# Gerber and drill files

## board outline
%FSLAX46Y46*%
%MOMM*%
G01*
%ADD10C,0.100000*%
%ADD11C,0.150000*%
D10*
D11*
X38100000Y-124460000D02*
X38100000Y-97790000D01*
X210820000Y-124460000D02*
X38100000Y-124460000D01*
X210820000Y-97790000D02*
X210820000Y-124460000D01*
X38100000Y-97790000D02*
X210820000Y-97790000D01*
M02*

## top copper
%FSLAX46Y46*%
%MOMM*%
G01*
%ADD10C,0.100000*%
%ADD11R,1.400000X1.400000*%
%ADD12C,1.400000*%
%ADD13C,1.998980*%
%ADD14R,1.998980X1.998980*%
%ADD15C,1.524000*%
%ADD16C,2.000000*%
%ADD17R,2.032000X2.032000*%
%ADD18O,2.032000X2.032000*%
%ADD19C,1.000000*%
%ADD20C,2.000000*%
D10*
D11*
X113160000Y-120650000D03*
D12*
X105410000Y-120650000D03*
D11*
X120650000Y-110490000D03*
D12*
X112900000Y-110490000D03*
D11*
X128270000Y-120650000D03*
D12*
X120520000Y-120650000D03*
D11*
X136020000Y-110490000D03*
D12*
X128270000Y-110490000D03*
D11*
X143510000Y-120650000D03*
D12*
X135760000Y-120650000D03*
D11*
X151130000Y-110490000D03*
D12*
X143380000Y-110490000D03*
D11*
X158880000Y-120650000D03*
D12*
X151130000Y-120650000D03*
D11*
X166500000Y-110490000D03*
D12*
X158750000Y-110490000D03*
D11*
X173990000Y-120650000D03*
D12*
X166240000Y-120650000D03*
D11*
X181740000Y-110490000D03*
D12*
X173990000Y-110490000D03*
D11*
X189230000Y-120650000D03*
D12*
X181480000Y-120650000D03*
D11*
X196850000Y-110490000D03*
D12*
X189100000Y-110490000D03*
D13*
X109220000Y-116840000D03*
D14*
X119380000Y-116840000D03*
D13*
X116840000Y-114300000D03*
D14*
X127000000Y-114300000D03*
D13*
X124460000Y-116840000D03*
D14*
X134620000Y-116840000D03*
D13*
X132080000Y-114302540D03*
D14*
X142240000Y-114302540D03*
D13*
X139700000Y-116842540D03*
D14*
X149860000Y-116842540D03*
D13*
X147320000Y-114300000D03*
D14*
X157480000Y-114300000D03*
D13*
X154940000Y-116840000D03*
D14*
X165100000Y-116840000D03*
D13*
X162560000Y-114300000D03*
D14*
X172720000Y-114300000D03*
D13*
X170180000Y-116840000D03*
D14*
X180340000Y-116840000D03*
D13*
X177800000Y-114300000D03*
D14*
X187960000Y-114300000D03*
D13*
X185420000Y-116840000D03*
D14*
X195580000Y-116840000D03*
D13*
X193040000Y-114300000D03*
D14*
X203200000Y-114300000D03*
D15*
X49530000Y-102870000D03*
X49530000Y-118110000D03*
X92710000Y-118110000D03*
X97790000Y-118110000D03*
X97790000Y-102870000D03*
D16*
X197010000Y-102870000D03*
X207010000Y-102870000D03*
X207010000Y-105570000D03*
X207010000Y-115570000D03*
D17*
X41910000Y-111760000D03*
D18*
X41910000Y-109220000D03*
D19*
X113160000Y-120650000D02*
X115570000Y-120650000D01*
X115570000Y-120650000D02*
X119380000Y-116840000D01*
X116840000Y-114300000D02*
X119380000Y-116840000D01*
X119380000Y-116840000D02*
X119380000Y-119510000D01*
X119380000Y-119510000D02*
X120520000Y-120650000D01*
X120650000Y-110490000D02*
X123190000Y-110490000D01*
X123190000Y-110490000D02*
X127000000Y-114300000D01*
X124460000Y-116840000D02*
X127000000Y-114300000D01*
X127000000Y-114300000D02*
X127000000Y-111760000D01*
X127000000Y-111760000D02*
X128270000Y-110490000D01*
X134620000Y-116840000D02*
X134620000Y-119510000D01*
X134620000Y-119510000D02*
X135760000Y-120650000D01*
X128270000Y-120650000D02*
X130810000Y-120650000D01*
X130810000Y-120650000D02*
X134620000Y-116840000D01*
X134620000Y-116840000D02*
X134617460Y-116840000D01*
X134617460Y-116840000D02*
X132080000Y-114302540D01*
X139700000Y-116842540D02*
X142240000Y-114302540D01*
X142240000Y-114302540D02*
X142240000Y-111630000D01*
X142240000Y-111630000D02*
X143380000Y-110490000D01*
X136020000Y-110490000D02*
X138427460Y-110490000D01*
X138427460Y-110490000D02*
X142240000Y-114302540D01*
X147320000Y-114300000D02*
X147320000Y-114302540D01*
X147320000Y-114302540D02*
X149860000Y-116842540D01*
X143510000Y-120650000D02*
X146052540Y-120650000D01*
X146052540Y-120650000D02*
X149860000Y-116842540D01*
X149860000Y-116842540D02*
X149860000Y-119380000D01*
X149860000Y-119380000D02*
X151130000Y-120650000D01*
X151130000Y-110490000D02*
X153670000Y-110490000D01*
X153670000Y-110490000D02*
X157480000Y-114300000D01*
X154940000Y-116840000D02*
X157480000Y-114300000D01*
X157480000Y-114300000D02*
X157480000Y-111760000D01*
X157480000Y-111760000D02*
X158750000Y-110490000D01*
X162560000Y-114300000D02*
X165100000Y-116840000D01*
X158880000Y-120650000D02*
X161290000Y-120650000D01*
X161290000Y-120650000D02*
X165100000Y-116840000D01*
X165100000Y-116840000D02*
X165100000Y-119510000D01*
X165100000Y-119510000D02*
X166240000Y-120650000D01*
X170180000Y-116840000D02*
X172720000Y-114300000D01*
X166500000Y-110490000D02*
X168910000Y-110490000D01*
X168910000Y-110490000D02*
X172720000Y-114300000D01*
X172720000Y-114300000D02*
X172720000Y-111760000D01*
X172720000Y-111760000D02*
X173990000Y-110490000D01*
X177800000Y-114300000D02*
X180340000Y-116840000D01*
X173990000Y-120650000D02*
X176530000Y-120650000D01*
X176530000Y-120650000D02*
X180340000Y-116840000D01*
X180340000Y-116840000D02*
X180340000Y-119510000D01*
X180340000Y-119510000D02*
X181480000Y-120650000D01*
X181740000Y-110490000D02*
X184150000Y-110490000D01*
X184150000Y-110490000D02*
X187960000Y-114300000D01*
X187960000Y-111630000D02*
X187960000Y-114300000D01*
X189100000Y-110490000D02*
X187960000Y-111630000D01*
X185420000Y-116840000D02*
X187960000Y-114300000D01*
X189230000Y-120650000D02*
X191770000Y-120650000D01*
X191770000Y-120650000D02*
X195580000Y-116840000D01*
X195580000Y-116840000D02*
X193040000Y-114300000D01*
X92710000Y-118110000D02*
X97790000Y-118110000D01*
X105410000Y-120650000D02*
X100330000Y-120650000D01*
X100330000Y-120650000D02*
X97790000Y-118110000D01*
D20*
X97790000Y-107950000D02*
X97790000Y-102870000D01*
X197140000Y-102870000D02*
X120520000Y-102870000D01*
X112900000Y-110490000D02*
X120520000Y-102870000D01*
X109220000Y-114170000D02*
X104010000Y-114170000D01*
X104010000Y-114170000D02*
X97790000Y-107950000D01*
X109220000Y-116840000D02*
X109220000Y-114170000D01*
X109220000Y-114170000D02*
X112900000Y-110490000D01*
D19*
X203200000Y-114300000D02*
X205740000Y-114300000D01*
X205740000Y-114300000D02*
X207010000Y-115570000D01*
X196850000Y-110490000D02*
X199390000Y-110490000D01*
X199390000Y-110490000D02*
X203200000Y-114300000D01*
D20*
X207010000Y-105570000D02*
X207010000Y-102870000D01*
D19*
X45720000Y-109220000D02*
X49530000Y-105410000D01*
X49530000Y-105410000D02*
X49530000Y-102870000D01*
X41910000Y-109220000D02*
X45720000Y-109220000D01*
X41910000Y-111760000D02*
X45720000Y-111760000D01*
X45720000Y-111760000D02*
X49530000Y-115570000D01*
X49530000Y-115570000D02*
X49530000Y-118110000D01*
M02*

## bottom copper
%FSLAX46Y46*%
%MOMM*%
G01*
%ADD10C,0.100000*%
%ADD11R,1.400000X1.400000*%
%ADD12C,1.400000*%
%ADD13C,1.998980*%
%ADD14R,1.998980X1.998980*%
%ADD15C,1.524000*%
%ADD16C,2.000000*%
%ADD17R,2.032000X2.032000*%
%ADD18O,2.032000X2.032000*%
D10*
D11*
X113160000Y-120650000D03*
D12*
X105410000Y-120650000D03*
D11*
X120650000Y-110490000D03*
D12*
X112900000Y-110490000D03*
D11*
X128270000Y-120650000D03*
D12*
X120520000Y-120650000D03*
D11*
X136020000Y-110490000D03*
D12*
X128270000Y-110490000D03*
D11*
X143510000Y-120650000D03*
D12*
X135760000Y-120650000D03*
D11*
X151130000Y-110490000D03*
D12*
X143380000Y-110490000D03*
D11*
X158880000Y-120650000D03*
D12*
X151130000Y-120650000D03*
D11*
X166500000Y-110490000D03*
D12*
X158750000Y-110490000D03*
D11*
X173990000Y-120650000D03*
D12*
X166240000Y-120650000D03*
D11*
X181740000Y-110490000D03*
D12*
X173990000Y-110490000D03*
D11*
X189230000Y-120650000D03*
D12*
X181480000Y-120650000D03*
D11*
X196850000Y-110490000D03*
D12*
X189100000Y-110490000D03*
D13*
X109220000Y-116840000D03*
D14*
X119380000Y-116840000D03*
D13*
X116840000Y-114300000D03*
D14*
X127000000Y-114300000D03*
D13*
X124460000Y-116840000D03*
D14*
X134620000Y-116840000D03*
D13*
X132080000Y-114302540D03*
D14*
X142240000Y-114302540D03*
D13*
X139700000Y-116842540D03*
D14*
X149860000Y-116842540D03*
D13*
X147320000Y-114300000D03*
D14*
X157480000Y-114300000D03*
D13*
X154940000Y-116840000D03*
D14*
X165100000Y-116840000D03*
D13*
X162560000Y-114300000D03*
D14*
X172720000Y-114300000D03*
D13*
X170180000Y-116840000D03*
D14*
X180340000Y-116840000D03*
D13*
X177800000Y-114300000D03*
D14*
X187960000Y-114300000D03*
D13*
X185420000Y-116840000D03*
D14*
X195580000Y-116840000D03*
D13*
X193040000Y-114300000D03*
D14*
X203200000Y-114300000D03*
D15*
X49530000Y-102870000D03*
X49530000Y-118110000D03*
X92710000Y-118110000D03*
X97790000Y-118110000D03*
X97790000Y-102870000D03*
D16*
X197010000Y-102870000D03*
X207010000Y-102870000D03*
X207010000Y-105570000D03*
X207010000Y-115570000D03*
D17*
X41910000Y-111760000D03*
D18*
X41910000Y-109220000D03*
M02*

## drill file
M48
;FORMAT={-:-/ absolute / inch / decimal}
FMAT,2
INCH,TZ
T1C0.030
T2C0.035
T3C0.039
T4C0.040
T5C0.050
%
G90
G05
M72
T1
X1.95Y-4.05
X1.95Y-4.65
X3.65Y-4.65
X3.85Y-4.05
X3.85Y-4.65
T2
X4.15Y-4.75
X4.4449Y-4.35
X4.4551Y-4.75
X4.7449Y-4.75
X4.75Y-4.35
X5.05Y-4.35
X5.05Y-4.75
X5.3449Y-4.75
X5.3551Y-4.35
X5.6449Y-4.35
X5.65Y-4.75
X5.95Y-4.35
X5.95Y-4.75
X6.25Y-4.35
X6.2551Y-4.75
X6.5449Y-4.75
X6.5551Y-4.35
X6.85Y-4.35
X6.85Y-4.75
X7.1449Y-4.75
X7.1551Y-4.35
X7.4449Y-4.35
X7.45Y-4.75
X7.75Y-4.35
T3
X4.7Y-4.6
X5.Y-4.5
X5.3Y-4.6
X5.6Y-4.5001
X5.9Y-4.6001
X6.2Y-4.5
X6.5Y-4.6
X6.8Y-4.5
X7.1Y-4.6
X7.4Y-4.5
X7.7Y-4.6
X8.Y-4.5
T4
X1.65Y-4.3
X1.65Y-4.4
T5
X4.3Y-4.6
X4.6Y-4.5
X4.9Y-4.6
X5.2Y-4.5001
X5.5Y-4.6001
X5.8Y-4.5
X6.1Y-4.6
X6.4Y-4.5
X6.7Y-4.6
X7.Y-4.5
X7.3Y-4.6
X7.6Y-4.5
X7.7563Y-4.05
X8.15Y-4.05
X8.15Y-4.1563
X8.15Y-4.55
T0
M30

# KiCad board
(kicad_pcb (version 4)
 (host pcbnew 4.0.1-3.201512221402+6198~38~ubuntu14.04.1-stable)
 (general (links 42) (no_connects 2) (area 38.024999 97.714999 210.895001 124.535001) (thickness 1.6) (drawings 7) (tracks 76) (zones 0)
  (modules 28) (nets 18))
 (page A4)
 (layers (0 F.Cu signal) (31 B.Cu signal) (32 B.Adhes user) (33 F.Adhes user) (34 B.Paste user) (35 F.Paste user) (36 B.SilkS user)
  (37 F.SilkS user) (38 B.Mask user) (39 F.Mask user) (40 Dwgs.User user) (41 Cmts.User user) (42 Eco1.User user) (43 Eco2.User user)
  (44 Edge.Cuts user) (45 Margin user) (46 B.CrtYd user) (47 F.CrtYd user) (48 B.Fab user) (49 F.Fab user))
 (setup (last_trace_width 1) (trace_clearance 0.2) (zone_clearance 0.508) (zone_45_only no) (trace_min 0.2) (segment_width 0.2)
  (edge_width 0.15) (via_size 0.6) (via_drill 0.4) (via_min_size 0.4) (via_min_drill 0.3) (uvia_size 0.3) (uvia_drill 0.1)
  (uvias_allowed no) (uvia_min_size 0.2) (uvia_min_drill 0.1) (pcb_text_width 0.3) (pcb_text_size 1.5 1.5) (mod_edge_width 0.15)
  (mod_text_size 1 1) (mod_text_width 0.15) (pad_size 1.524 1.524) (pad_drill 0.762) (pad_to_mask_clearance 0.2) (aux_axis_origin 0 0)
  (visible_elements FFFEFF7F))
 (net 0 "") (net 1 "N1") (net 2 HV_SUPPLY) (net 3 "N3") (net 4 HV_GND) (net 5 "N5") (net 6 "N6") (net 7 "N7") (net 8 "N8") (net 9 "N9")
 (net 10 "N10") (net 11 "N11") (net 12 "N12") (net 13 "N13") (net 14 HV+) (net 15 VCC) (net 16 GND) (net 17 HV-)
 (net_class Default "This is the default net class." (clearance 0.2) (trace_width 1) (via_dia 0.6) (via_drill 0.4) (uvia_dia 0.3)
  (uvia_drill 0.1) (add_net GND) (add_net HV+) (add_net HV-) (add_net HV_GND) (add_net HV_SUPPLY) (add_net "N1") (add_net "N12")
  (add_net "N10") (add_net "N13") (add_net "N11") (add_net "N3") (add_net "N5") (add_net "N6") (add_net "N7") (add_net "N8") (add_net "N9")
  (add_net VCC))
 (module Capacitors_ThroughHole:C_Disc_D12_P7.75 (layer F.Cu) (at 113.16 120.65 180)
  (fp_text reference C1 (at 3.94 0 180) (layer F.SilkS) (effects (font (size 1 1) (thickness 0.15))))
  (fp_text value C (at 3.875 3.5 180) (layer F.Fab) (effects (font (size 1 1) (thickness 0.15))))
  (pad 1 thru_hole rect (at 0 0 180) (size 1.4 1.4) (drill 0.9) (layers *.Cu *.Mask F.SilkS) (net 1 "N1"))
  (pad 2 thru_hole circle (at 7.75 0 180) (size 1.4 1.4) (drill 0.9) (layers *.Cu *.Mask F.SilkS) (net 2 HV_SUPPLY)))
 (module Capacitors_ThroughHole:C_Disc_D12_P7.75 (layer F.Cu) (at 120.65 110.49 180)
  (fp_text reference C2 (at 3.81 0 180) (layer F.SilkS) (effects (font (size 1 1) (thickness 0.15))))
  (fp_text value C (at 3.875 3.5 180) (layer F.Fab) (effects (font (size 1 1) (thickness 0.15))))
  (pad 1 thru_hole rect (at 0 0 180) (size 1.4 1.4) (drill 0.9) (layers *.Cu *.Mask F.SilkS) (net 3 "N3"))
  (pad 2 thru_hole circle (at 7.75 0 180) (size 1.4 1.4) (drill 0.9) (layers *.Cu *.Mask F.SilkS) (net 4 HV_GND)))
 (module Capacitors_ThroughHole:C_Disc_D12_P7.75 (layer F.Cu) (at 128.27 120.65 180)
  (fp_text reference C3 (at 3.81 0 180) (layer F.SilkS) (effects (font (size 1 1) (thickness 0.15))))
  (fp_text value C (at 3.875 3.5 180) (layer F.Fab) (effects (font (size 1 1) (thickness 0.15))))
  (pad 1 thru_hole rect (at 0 0 180) (size 1.4 1.4) (drill 0.9) (layers *.Cu *.Mask F.SilkS) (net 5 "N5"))
  (pad 2 thru_hole circle (at 7.75 0 180) (size 1.4 1.4) (drill 0.9) (layers *.Cu *.Mask F.SilkS) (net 1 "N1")))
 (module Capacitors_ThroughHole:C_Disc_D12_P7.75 (layer F.Cu) (at 136.02 110.49 180)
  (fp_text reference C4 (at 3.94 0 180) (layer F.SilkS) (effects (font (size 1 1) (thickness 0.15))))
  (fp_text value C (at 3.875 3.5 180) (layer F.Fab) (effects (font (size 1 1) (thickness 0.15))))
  (pad 1 thru_hole rect (at 0 0 180) (size 1.4 1.4) (drill 0.9) (layers *.Cu *.Mask F.SilkS) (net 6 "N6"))
  (pad 2 thru_hole circle (at 7.75 0 180) (size 1.4 1.4) (drill 0.9) (layers *.Cu *.Mask F.SilkS) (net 3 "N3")))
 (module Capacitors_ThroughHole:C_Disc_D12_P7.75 (layer F.Cu) (at 143.51 120.65 180)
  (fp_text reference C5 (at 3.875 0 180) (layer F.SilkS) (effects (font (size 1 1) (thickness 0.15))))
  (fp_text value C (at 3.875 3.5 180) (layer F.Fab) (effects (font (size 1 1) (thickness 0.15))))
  (pad 1 thru_hole rect (at 0 0 180) (size 1.4 1.4) (drill 0.9) (layers *.Cu *.Mask F.SilkS) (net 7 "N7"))
  (pad 2 thru_hole circle (at 7.75 0 180) (size 1.4 1.4) (drill 0.9) (layers *.Cu *.Mask F.SilkS) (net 5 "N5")))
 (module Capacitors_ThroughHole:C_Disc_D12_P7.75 (layer F.Cu) (at 151.13 110.49 180)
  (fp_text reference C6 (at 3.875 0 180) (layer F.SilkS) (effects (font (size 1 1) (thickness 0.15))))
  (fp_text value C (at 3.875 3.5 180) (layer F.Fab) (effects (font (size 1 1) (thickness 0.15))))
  (pad 1 thru_hole rect (at 0 0 180) (size 1.4 1.4) (drill 0.9) (layers *.Cu *.Mask F.SilkS) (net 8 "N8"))
  (pad 2 thru_hole circle (at 7.75 0 180) (size 1.4 1.4) (drill 0.9) (layers *.Cu *.Mask F.SilkS) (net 6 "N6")))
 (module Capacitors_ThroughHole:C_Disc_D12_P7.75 (layer F.Cu) (at 158.88 120.65 180)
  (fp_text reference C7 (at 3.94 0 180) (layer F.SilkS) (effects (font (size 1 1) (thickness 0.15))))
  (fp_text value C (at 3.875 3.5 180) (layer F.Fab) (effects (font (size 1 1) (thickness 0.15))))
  (pad 1 thru_hole rect (at 0 0 180) (size 1.4 1.4) (drill 0.9) (layers *.Cu *.Mask F.SilkS) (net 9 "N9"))
  (pad 2 thru_hole circle (at 7.75 0 180) (size 1.4 1.4) (drill 0.9) (layers *.Cu *.Mask F.SilkS) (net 7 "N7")))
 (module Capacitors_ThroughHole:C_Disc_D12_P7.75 (layer F.Cu) (at 166.5 110.49 180)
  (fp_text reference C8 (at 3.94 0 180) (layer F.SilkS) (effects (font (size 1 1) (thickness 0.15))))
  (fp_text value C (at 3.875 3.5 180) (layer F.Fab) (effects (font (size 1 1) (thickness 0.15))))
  (pad 1 thru_hole rect (at 0 0 180) (size 1.4 1.4) (drill 0.9) (layers *.Cu *.Mask F.SilkS) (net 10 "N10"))
  (pad 2 thru_hole circle (at 7.75 0 180) (size 1.4 1.4) (drill 0.9) (layers *.Cu *.Mask F.SilkS) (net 8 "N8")))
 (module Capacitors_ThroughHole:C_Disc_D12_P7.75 (layer F.Cu) (at 173.99 120.65 180)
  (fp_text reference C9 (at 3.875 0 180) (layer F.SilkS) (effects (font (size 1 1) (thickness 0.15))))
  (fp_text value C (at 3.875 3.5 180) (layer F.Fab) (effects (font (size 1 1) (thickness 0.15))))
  (pad 1 thru_hole rect (at 0 0 180) (size 1.4 1.4) (drill 0.9) (layers *.Cu *.Mask F.SilkS) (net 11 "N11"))
  (pad 2 thru_hole circle (at 7.75 0 180) (size 1.4 1.4) (drill 0.9) (layers *.Cu *.Mask F.SilkS) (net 9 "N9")))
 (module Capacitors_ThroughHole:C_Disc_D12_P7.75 (layer F.Cu) (at 181.74 110.49 180)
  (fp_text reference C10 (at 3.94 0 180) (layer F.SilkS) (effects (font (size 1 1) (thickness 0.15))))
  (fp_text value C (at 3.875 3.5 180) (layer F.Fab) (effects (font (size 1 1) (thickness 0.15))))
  (pad 1 thru_hole rect (at 0 0 180) (size 1.4 1.4) (drill 0.9) (layers *.Cu *.Mask F.SilkS) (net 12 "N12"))
  (pad 2 thru_hole circle (at 7.75 0 180) (size 1.4 1.4) (drill 0.9) (layers *.Cu *.Mask F.SilkS) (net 10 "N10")))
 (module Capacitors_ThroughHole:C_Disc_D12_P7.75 (layer F.Cu) (at 189.23 120.65 180)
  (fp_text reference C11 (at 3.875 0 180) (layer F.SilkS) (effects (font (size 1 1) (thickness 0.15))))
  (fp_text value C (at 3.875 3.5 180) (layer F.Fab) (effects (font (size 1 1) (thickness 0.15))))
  (pad 1 thru_hole rect (at 0 0 180) (size 1.4 1.4) (drill 0.9) (layers *.Cu *.Mask F.SilkS) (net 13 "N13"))
  (pad 2 thru_hole circle (at 7.75 0 180) (size 1.4 1.4) (drill 0.9) (layers *.Cu *.Mask F.SilkS) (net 11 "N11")))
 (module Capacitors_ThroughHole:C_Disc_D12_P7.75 (layer F.Cu) (at 196.85 110.49 180)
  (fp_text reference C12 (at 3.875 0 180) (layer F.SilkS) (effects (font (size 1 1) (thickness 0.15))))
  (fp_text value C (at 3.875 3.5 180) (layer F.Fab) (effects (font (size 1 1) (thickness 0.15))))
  (pad 1 thru_hole rect (at 0 0 180) (size 1.4 1.4) (drill 0.9) (layers *.Cu *.Mask F.SilkS) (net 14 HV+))
  (pad 2 thru_hole circle (at 7.75 0 180) (size 1.4 1.4) (drill 0.9) (layers *.Cu *.Mask F.SilkS) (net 12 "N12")))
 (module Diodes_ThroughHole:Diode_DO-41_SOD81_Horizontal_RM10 (layer F.Cu) (at 119.38 116.83746 180)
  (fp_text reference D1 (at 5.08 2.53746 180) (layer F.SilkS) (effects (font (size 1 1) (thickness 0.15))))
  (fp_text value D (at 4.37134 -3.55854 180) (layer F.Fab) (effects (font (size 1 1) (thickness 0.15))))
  (pad 2 thru_hole circle (at 10.16 -0.00254) (size 1.99898 1.99898) (drill 1.27) (layers *.Cu *.Mask F.SilkS) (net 4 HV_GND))
  (pad 1 thru_hole rect (at 0 -0.00254) (size 1.99898 1.99898) (drill 1.00076) (layers *.Cu *.Mask F.SilkS) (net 1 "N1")))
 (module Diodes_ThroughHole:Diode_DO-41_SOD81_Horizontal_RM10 (layer F.Cu) (at 127 114.29746 180)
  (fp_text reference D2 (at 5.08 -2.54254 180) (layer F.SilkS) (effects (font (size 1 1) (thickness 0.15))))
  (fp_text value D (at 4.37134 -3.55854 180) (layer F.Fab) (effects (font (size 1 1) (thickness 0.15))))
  (pad 2 thru_hole circle (at 10.16 -0.00254) (size 1.99898 1.99898) (drill 1.27) (layers *.Cu *.Mask F.SilkS) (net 1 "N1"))
  (pad 1 thru_hole rect (at 0 -0.00254) (size 1.99898 1.99898) (drill 1.00076) (layers *.Cu *.Mask F.SilkS) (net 3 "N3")))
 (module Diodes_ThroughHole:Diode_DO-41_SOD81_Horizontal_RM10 (layer F.Cu) (at 134.62 116.83746 180)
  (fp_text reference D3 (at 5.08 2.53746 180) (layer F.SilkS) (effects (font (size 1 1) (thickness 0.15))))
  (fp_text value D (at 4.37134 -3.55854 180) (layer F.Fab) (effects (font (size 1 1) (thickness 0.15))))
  (pad 2 thru_hole circle (at 10.16 -0.00254) (size 1.99898 1.99898) (drill 1.27) (layers *.Cu *.Mask F.SilkS) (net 3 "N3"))
  (pad 1 thru_hole rect (at 0 -0.00254) (size 1.99898 1.99898) (drill 1.00076) (layers *.Cu *.Mask F.SilkS) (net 5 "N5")))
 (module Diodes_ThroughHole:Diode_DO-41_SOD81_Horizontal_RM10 (layer F.Cu) (at 142.24 114.3 180)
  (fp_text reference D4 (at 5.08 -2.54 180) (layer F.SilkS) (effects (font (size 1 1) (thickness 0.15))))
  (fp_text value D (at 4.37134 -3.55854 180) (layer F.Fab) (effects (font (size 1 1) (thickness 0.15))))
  (pad 2 thru_hole circle (at 10.16 -0.00254) (size 1.99898 1.99898) (drill 1.27) (layers *.Cu *.Mask F.SilkS) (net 5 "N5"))
  (pad 1 thru_hole rect (at 0 -0.00254) (size 1.99898 1.99898) (drill 1.00076) (layers *.Cu *.Mask F.SilkS) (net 6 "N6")))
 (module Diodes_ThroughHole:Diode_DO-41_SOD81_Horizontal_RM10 (layer F.Cu) (at 149.86 116.84 180)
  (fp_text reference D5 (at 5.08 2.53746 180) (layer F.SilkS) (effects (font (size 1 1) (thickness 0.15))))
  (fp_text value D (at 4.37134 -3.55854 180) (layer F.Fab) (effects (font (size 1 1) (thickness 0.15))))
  (pad 2 thru_hole circle (at 10.16 -0.00254) (size 1.99898 1.99898) (drill 1.27) (layers *.Cu *.Mask F.SilkS) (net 6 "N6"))
  (pad 1 thru_hole rect (at 0 -0.00254) (size 1.99898 1.99898) (drill 1.00076) (layers *.Cu *.Mask F.SilkS) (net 7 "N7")))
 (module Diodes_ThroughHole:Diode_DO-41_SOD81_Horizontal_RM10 (layer F.Cu) (at 157.48 114.29746 180)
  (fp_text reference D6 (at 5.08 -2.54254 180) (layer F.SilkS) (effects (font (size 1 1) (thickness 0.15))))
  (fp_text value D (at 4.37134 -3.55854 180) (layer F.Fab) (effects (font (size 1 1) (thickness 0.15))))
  (pad 2 thru_hole circle (at 10.16 -0.00254) (size 1.99898 1.99898) (drill 1.27) (layers *.Cu *.Mask F.SilkS) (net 7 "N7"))
  (pad 1 thru_hole rect (at 0 -0.00254) (size 1.99898 1.99898) (drill 1.00076) (layers *.Cu *.Mask F.SilkS) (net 8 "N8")))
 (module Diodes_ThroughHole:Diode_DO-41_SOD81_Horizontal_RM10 (layer F.Cu) (at 165.1 116.83746 180)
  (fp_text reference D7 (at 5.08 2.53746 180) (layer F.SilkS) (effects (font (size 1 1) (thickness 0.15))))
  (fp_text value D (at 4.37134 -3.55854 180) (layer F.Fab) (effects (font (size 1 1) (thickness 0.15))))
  (pad 2 thru_hole circle (at 10.16 -0.00254) (size 1.99898 1.99898) (drill 1.27) (layers *.Cu *.Mask F.SilkS) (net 8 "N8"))
  (pad 1 thru_hole rect (at 0 -0.00254) (size 1.99898 1.99898) (drill 1.00076) (layers *.Cu *.Mask F.SilkS) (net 9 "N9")))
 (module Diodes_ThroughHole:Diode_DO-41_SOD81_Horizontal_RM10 (layer F.Cu) (at 172.72 114.29746 180)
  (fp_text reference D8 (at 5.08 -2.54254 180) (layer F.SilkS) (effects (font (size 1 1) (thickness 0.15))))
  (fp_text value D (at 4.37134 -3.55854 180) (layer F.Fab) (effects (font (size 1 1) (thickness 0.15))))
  (pad 2 thru_hole circle (at 10.16 -0.00254) (size 1.99898 1.99898) (drill 1.27) (layers *.Cu *.Mask F.SilkS) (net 9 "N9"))
  (pad 1 thru_hole rect (at 0 -0.00254) (size 1.99898 1.99898) (drill 1.00076) (layers *.Cu *.Mask F.SilkS) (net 10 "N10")))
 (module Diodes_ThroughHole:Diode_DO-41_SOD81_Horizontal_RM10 (layer F.Cu) (at 180.34 116.83746 180)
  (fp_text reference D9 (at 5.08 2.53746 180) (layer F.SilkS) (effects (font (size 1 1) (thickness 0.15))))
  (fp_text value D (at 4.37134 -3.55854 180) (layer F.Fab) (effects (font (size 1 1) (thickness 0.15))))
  (pad 2 thru_hole circle (at 10.16 -0.00254) (size 1.99898 1.99898) (drill 1.27) (layers *.Cu *.Mask F.SilkS) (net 10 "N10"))
  (pad 1 thru_hole rect (at 0 -0.00254) (size 1.99898 1.99898) (drill 1.00076) (layers *.Cu *.Mask F.SilkS) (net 11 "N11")))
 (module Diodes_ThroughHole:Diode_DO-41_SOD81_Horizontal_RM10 (layer F.Cu) (at 187.96 114.29746 180)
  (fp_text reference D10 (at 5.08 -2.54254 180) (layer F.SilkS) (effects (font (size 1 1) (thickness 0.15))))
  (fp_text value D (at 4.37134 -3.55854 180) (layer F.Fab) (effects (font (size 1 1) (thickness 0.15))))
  (pad 2 thru_hole circle (at 10.16 -0.00254) (size 1.99898 1.99898) (drill 1.27) (layers *.Cu *.Mask F.SilkS) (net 11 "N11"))
  (pad 1 thru_hole rect (at 0 -0.00254) (size 1.99898 1.99898) (drill 1.00076) (layers *.Cu *.Mask F.SilkS) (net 12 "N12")))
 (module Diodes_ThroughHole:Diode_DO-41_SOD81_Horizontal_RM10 (layer F.Cu) (at 195.58 116.83746 180)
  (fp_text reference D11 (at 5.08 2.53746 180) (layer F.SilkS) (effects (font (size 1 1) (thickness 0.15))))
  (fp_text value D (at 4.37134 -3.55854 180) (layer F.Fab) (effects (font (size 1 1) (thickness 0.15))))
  (pad 2 thru_hole circle (at 10.16 -0.00254) (size 1.99898 1.99898) (drill 1.27) (layers *.Cu *.Mask F.SilkS) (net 12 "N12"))
  (pad 1 thru_hole rect (at 0 -0.00254) (size 1.99898 1.99898) (drill 1.00076) (layers *.Cu *.Mask F.SilkS) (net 13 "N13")))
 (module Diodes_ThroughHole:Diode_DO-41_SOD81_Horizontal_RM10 (layer F.Cu) (at 203.2 114.29746 180)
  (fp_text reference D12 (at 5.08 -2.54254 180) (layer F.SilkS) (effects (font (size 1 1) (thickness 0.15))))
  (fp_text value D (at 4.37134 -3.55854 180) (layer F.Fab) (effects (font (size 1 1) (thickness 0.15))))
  (pad 2 thru_hole circle (at 10.16 -0.00254) (size 1.99898 1.99898) (drill 1.27) (layers *.Cu *.Mask F.SilkS) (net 13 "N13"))
  (pad 1 thru_hole rect (at 0 -0.00254) (size 1.99898 1.99898) (drill 1.00076) (layers *.Cu *.Mask F.SilkS) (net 14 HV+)))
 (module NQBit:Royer (layer F.Cu) (at 74.93 110.49)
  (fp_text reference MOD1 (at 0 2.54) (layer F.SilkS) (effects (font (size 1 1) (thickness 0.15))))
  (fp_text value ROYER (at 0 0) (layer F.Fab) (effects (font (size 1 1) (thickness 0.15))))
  (pad 1 thru_hole circle (at -25.4 -7.62) (size 1.524 1.524) (drill 0.762) (layers *.Cu *.Mask F.SilkS) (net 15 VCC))
  (pad 2 thru_hole circle (at -25.4 7.62) (size 1.524 1.524) (drill 0.762) (layers *.Cu *.Mask F.SilkS) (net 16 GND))
  (pad 3 thru_hole circle (at 17.78 7.62) (size 1.524 1.524) (drill 0.762) (layers *.Cu *.Mask F.SilkS) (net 2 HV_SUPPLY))
  (pad 4 thru_hole circle (at 22.86 7.62) (size 1.524 1.524) (drill 0.762) (layers *.Cu *.Mask F.SilkS) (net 2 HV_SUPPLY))
  (pad 5 thru_hole circle (at 22.86 -7.62) (size 1.524 1.524) (drill 0.762) (layers *.Cu *.Mask F.SilkS) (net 4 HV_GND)))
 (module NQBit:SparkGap (layer F.Cu) (at 197.01 102.87)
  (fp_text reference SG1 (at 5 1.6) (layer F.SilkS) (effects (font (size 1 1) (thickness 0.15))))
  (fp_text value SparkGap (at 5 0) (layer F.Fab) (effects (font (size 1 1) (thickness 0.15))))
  (pad 1 thru_hole circle (at 0 0) (size 2 2) (drill 1.27) (layers *.Cu *.Mask F.SilkS) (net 4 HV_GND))
  (pad 2 thru_hole circle (at 10 0) (size 2 2) (drill 1.27) (layers *.Cu *.Mask F.SilkS) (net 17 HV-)))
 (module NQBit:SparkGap (layer F.Cu) (at 207.01 105.57 270)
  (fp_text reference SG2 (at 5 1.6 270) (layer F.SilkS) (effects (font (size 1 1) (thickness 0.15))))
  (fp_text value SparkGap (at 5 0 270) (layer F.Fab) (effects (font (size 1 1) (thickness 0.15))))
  (pad 1 thru_hole circle (at 0 0 270) (size 2 2) (drill 1.27) (layers *.Cu *.Mask F.SilkS) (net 17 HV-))
  (pad 2 thru_hole circle (at 10 0 270) (size 2 2) (drill 1.27) (layers *.Cu *.Mask F.SilkS) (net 14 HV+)))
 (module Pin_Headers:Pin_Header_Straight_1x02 (layer F.Cu) (at 41.91 111.76 180)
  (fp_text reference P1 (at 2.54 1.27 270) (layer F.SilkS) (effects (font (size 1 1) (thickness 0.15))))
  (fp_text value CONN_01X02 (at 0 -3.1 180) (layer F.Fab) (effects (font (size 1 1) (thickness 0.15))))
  (pad 1 thru_hole rect (at 0 0 180) (size 2.032 2.032) (drill 1.016) (layers *.Cu *.Mask F.SilkS) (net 16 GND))
  (pad 2 thru_hole oval (at 0 2.54 180) (size 2.032 2.032) (drill 1.016) (layers *.Cu *.Mask F.SilkS) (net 15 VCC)))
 (gr_line (start 38.1 124.46) (end 38.1 97.79) (layer Edge.Cuts) (width 0.15))
 (gr_line (start 210.82 124.46) (end 38.1 124.46) (layer Edge.Cuts) (width 0.15))
 (gr_line (start 210.82 97.79) (end 210.82 124.46) (layer Edge.Cuts) (width 0.15))
 (gr_line (start 38.1 97.79) (end 210.82 97.79) (layer Edge.Cuts) (width 0.15))
 (segment (start 113.16 120.65) (end 115.57 120.65) (width 1) (layer F.Cu) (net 1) (status 10))
 (segment (start 115.57 120.65) (end 119.38 116.84) (width 1) (layer F.Cu) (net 1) (status 20))
 (segment (start 116.84 114.3) (end 119.38 116.84) (width 1) (layer F.Cu) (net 1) (status 30))
 (segment (start 119.38 116.84) (end 119.38 119.51) (width 1) (layer F.Cu) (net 1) (status 10))
 (segment (start 119.38 119.51) (end 120.52 120.65) (width 1) (layer F.Cu) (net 1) (status 20))
 (segment (start 120.65 110.49) (end 123.19 110.49) (width 1) (layer F.Cu) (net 3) (status 10))
 (segment (start 123.19 110.49) (end 127 114.3) (width 1) (layer F.Cu) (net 3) (status 20))
 (segment (start 124.46 116.84) (end 127 114.3) (width 1) (layer F.Cu) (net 3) (status 30))
 (segment (start 127 114.3) (end 127 111.76) (width 1) (layer F.Cu) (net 3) (status 10))
 (segment (start 127 111.76) (end 128.27 110.49) (width 1) (layer F.Cu) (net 3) (status 20))
 (segment (start 134.62 116.84) (end 134.62 119.51) (width 1) (layer F.Cu) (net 5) (status 10))
 (segment (start 134.62 119.51) (end 135.76 120.65) (width 1) (layer F.Cu) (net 5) (status 20))
 (segment (start 128.27 120.65) (end 130.81 120.65) (width 1) (layer F.Cu) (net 5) (status 10))
 (segment (start 130.81 120.65) (end 134.62 116.84) (width 1) (layer F.Cu) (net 5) (status 20))
 (segment (start 134.62 116.84) (end 134.61746 116.84) (width 1) (layer F.Cu) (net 5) (status 30))
 (segment (start 134.61746 116.84) (end 132.08 114.30254) (width 1) (layer F.Cu) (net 5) (status 30))
 (segment (start 139.7 116.84254) (end 142.24 114.30254) (width 1) (layer F.Cu) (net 6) (status 30))
 (segment (start 142.24 114.30254) (end 142.24 111.63) (width 1) (layer F.Cu) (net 6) (status 10))
 (segment (start 142.24 111.63) (end 143.38 110.49) (width 1) (layer F.Cu) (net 6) (status 20))
 (segment (start 136.02 110.49) (end 138.42746 110.49) (width 1) (layer F.Cu) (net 6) (status 10))
 (segment (start 138.42746 110.49) (end 142.24 114.30254) (width 1) (layer F.Cu) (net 6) (status 20))
 (segment (start 147.32 114.3) (end 147.32 114.30254) (width 1) (layer F.Cu) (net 7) (status 30))
 (segment (start 147.32 114.30254) (end 149.86 116.84254) (width 1) (layer F.Cu) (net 7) (status 30))
 (segment (start 143.51 120.65) (end 146.05254 120.65) (width 1) (layer F.Cu) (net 7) (status 10))
 (segment (start 146.05254 120.65) (end 149.86 116.84254) (width 1) (layer F.Cu) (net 7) (status 20))
 (segment (start 149.86 116.84254) (end 149.86 119.38) (width 1) (layer F.Cu) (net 7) (status 10))
 (segment (start 149.86 119.38) (end 151.13 120.65) (width 1) (layer F.Cu) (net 7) (status 20))
 (segment (start 151.13 110.49) (end 153.67 110.49) (width 1) (layer F.Cu) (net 8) (status 10))
 (segment (start 153.67 110.49) (end 157.48 114.3) (width 1) (layer F.Cu) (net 8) (status 20))
 (segment (start 154.94 116.84) (end 157.48 114.3) (width 1) (layer F.Cu) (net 8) (status 30))
 (segment (start 157.48 114.3) (end 157.48 111.76) (width 1) (layer F.Cu) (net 8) (status 10))
 (segment (start 157.48 111.76) (end 158.75 110.49) (width 1) (layer F.Cu) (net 8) (status 20))
 (segment (start 162.56 114.3) (end 165.1 116.84) (width 1) (layer F.Cu) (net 9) (status 30))
 (segment (start 158.88 120.65) (end 161.29 120.65) (width 1) (layer F.Cu) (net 9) (status 10))
 (segment (start 161.29 120.65) (end 165.1 116.84) (width 1) (layer F.Cu) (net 9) (status 20))
 (segment (start 165.1 116.84) (end 165.1 119.51) (width 1) (layer F.Cu) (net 9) (status 10))
 (segment (start 165.1 119.51) (end 166.24 120.65) (width 1) (layer F.Cu) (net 9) (status 20))
 (segment (start 170.18 116.84) (end 172.72 114.3) (width 1) (layer F.Cu) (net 10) (status 30))
 (segment (start 166.5 110.49) (end 168.91 110.49) (width 1) (layer F.Cu) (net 10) (status 10))
 (segment (start 168.91 110.49) (end 172.72 114.3) (width 1) (layer F.Cu) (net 10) (status 20))
 (segment (start 172.72 114.3) (end 172.72 111.76) (width 1) (layer F.Cu) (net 10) (status 10))
 (segment (start 172.72 111.76) (end 173.99 110.49) (width 1) (layer F.Cu) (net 10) (status 20))
 (segment (start 177.8 114.3) (end 180.34 116.84) (width 1) (layer F.Cu) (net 11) (status 30))
 (segment (start 173.99 120.65) (end 176.53 120.65) (width 1) (layer F.Cu) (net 11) (status 10))
 (segment (start 176.53 120.65) (end 180.34 116.84) (width 1) (layer F.Cu) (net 11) (status 20))
 (segment (start 180.34 116.84) (end 180.34 119.51) (width 1) (layer F.Cu) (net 11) (status 10))
 (segment (start 180.34 119.51) (end 181.48 120.65) (width 1) (layer F.Cu) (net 11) (status 20))
 (segment (start 181.74 110.49) (end 184.15 110.49) (width 1) (layer F.Cu) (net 12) (status 10))
 (segment (start 184.15 110.49) (end 187.96 114.3) (width 1) (layer F.Cu) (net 12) (status 20))
 (segment (start 187.96 111.63) (end 187.96 114.3) (width 1) (layer F.Cu) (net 12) (status 20))
 (segment (start 189.1 110.49) (end 187.96 111.63) (width 1) (layer F.Cu) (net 12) (status 10))
 (segment (start 185.42 116.84) (end 187.96 114.3) (width 1) (layer F.Cu) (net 12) (status 30))
 (segment (start 189.23 120.65) (end 191.77 120.65) (width 1) (layer F.Cu) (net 13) (status 10))
 (segment (start 191.77 120.65) (end 195.58 116.84) (width 1) (layer F.Cu) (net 13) (status 20))
 (segment (start 195.58 116.84) (end 193.04 114.3) (width 1) (layer F.Cu) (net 13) (status 30))
 (segment (start 92.71 118.11) (end 97.79 118.11) (width 1) (layer F.Cu) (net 2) (status 30))
 (segment (start 105.41 120.65) (end 100.33 120.65) (width 1) (layer F.Cu) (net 2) (status 10))
 (segment (start 100.33 120.65) (end 97.79 118.11) (width 1) (layer F.Cu) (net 2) (status 20))
 (segment (start 97.79 107.95) (end 97.79 102.87) (width 2) (layer F.Cu) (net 4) (status 20))
 (segment (start 197.14 102.87) (end 120.52 102.87) (width 2) (layer F.Cu) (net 4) (status 10))
 (segment (start 112.9 110.49) (end 120.52 102.87) (width 2) (layer F.Cu) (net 4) (status 10))
 (segment (start 109.22 114.17) (end 104.01 114.17) (width 2) (layer F.Cu) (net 4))
 (segment (start 104.01 114.17) (end 97.79 107.95) (width 2) (layer F.Cu) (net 4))
 (segment (start 109.22 116.84) (end 109.22 114.17) (width 2) (layer F.Cu) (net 4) (status 10))
 (segment (start 109.22 114.17) (end 112.9 110.49) (width 2) (layer F.Cu) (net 4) (status 20))
 (segment (start 203.2 114.3) (end 205.74 114.3) (width 1) (layer F.Cu) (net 14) (status 10))
 (segment (start 205.74 114.3) (end 207.01 115.57) (width 1) (layer F.Cu) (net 14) (status 20))
 (segment (start 196.85 110.49) (end 199.39 110.49) (width 1) (layer F.Cu) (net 14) (status 10))
 (segment (start 199.39 110.49) (end 203.2 114.3) (width 1) (layer F.Cu) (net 14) (status 20))
 (segment (start 207.01 105.57) (end 207.01 102.87) (width 2) (layer F.Cu) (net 17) (status 30))
 (segment (start 45.72 109.22) (end 49.53 105.41) (width 1) (layer F.Cu) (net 15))
 (segment (start 49.53 105.41) (end 49.53 102.87) (width 1) (layer F.Cu) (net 15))
 (segment (start 41.91 109.22) (end 45.72 109.22) (width 1) (layer F.Cu) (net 15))
 (segment (start 41.91 111.76) (end 45.72 111.76) (width 1) (layer F.Cu) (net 16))
 (segment (start 45.72 111.76) (end 49.53 115.57) (width 1) (layer F.Cu) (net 16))
 (segment (start 49.53 115.57) (end 49.53 118.11) (width 1) (layer F.Cu) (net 16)))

